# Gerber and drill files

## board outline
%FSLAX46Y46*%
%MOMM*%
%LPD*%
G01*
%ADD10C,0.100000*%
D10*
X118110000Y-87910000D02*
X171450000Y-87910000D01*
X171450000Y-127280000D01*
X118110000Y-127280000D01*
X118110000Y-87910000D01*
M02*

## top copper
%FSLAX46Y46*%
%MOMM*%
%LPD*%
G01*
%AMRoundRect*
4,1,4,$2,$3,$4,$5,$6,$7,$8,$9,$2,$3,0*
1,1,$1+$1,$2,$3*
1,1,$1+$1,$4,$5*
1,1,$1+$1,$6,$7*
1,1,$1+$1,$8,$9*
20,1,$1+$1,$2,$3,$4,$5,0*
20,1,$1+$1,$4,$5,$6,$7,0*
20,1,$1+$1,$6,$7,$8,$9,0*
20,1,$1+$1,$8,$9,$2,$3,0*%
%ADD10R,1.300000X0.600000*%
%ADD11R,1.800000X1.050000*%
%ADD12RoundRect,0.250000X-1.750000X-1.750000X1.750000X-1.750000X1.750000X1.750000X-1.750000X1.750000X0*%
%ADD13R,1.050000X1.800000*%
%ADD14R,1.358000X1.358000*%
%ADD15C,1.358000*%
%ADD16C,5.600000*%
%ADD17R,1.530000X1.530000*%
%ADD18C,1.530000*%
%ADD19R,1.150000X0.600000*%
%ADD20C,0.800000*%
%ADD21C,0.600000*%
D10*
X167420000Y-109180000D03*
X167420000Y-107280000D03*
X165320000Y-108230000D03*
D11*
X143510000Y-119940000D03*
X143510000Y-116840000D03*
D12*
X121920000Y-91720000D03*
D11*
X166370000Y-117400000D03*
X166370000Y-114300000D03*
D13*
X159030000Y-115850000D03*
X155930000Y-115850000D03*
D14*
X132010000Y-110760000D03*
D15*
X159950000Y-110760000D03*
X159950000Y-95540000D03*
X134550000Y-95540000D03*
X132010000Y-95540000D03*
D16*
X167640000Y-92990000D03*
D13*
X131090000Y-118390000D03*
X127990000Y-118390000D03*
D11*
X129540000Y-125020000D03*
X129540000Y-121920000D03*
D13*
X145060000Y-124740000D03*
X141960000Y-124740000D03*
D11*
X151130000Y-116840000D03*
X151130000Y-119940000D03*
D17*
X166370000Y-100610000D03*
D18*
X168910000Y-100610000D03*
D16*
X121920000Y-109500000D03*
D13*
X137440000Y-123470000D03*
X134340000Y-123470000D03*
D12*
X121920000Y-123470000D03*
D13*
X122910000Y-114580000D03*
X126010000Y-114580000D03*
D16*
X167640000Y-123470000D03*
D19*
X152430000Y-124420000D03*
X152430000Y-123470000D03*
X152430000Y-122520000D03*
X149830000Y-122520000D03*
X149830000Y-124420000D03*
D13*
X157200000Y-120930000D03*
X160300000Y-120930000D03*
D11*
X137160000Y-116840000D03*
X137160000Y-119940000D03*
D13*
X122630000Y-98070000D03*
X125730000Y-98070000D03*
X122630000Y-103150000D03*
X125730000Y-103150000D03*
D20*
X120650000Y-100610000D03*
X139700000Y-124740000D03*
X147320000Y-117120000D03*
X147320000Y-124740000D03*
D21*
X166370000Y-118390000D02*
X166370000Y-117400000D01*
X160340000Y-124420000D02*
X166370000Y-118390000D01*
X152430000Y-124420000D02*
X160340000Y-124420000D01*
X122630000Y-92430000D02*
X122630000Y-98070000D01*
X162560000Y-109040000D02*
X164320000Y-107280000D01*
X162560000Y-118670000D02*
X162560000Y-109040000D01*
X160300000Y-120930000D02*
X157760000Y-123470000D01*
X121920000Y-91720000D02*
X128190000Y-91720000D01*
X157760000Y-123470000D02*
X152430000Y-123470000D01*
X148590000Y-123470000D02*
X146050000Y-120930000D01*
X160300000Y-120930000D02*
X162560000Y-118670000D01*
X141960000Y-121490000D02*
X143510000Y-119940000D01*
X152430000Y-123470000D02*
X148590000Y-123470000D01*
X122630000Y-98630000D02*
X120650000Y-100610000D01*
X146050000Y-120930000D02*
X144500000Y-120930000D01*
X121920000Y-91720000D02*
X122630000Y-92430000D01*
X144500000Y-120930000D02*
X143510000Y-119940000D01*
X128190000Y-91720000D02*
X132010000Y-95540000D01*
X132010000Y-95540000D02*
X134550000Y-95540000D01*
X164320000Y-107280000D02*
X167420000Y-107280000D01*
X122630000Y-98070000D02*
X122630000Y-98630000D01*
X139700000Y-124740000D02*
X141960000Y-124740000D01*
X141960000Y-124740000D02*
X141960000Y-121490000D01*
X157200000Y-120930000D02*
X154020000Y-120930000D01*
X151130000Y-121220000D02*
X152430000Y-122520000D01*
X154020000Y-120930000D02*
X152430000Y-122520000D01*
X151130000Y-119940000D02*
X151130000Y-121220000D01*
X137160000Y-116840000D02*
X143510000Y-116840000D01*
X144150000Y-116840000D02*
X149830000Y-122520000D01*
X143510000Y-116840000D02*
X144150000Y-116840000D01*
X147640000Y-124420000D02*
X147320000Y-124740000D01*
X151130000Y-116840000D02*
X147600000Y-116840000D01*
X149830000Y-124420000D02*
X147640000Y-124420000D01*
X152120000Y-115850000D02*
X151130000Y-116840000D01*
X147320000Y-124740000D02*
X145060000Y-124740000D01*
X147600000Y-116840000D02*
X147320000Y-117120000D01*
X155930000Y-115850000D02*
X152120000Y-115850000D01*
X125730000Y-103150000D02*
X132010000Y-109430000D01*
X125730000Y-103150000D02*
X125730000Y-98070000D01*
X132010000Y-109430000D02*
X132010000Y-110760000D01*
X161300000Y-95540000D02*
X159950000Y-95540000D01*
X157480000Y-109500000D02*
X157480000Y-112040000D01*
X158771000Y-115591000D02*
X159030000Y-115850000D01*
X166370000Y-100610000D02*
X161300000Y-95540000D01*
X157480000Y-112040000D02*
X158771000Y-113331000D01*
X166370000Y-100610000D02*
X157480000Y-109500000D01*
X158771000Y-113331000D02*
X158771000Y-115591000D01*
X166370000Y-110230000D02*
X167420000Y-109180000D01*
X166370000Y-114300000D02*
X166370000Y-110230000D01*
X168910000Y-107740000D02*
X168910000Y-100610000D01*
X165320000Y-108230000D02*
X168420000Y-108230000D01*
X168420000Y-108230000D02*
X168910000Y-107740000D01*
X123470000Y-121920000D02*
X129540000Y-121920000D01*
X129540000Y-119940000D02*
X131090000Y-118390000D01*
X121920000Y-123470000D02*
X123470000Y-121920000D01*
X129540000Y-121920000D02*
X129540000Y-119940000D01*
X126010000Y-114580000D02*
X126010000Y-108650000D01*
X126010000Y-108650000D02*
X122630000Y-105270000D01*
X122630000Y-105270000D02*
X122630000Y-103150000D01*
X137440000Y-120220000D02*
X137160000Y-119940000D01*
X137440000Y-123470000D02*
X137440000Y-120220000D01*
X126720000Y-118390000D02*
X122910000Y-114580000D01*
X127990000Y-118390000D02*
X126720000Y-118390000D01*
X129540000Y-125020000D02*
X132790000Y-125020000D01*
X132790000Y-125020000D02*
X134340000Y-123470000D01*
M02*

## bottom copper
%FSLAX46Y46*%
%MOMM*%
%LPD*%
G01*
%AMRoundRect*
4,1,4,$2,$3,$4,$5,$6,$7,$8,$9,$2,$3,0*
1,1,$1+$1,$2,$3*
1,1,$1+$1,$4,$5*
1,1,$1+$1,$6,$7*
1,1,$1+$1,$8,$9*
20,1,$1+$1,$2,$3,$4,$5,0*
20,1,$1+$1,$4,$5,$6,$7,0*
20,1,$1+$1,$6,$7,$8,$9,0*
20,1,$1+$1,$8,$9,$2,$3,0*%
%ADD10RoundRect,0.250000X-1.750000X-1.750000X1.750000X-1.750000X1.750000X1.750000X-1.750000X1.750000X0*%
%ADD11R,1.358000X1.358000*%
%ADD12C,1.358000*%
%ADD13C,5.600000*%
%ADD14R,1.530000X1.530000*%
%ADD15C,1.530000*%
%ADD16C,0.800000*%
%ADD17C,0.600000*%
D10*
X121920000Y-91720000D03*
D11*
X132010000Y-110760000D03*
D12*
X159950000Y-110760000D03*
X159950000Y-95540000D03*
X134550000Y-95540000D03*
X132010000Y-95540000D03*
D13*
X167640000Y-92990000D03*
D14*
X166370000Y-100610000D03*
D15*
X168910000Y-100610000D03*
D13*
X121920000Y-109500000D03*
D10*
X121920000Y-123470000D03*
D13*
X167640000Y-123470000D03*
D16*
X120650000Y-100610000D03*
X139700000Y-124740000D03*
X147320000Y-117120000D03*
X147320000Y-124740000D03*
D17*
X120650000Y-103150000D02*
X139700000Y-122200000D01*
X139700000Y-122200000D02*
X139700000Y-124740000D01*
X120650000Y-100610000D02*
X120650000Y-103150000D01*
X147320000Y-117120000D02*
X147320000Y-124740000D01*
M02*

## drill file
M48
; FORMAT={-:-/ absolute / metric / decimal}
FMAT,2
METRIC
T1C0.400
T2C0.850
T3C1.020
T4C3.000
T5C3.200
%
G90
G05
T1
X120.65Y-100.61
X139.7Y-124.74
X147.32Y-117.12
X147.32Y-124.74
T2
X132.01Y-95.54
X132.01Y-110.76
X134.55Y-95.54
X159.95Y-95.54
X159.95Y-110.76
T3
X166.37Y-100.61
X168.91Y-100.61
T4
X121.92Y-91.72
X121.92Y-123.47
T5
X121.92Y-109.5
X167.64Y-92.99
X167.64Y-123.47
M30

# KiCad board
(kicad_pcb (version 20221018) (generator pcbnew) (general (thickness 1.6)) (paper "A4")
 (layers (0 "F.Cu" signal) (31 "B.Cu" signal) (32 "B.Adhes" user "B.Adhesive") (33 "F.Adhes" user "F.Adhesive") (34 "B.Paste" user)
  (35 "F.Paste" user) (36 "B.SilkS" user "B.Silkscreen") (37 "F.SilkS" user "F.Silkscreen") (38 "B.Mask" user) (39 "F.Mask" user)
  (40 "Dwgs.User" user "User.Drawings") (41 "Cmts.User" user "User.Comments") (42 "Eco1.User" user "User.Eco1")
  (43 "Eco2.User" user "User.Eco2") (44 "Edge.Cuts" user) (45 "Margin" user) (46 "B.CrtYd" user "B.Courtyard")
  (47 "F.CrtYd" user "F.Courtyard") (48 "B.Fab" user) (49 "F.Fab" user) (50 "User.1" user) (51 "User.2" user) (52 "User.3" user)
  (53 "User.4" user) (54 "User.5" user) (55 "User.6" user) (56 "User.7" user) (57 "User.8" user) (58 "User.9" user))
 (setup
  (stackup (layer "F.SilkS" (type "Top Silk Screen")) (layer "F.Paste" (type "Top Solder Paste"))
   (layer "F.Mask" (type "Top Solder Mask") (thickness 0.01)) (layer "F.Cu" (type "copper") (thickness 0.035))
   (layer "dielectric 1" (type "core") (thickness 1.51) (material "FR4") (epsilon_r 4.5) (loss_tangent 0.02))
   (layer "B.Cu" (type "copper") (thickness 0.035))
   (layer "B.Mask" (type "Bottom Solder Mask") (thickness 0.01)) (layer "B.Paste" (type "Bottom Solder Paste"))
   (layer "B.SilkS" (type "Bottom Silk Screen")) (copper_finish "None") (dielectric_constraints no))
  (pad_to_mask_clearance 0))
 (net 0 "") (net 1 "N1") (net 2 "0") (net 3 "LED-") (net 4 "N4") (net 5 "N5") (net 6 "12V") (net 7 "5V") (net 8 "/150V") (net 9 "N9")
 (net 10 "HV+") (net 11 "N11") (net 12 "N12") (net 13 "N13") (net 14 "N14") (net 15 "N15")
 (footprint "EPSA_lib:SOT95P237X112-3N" (layer "F.Cu") (at 166.37 108.23 180)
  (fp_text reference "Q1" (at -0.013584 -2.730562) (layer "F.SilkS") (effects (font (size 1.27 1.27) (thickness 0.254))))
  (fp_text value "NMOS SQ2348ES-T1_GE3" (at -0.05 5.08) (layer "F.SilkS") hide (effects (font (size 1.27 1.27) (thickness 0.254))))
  (pad "1" smd rect (at -1.05 -0.95 270) (size 0.6 1.3) (layers "F.Cu" "F.Paste" "F.Mask") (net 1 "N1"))
  (pad "2" smd rect (at -1.05 0.95 270) (size 0.6 1.3) (layers "F.Cu" "F.Paste" "F.Mask") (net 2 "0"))
  (pad "3" smd rect (at 1.05 0 270) (size 0.6 1.3) (layers "F.Cu" "F.Paste" "F.Mask") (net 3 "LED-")))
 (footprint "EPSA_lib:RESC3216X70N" (layer "F.Cu") (at 143.51 118.39 90)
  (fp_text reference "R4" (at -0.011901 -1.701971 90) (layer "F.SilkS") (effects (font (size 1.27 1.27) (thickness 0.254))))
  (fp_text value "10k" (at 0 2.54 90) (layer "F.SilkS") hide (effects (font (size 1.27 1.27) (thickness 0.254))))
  (pad "1" smd rect (at -1.55 0 90) (size 1.05 1.8) (layers "F.Cu" "F.Paste" "F.Mask") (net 2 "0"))
  (pad "2" smd rect (at 1.55 0 90) (size 1.05 1.8) (layers "F.Cu" "F.Paste" "F.Mask") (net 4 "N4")))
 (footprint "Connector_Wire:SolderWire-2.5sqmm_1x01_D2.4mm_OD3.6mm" (layer "F.Cu") (at 121.92 91.72)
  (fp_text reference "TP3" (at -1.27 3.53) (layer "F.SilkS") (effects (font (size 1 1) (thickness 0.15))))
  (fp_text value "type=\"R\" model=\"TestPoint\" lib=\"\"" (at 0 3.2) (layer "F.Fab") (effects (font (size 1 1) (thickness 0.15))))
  (pad "1" thru_hole roundrect (at 0 0) (size 4 4) (drill 3) (layers "*.Cu" "*.Mask") (roundrect_rratio 0.0625) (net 2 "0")))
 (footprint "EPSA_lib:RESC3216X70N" (layer "F.Cu") (at 166.37 115.85 90)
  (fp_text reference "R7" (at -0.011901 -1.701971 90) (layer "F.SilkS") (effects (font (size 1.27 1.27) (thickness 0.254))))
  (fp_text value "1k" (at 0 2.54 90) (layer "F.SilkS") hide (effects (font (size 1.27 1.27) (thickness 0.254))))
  (pad "1" smd rect (at -1.55 0 90) (size 1.05 1.8) (layers "F.Cu" "F.Paste" "F.Mask") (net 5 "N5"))
  (pad "2" smd rect (at 1.55 0 90) (size 1.05 1.8) (layers "F.Cu" "F.Paste" "F.Mask") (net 1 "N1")))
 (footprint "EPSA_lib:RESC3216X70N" (layer "F.Cu") (at 157.48 115.85 180)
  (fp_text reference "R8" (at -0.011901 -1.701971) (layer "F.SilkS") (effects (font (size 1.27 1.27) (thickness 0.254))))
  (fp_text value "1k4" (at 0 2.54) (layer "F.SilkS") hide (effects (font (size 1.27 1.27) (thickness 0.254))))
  (pad "1" smd rect (at -1.55 0 180) (size 1.05 1.8) (layers "F.Cu" "F.Paste" "F.Mask") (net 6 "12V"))
  (pad "2" smd rect (at 1.55 0 180) (size 1.05 1.8) (layers "F.Cu" "F.Paste" "F.Mask") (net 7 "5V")))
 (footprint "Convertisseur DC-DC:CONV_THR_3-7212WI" (layer "F.Cu") (at 146.05 103.15 180)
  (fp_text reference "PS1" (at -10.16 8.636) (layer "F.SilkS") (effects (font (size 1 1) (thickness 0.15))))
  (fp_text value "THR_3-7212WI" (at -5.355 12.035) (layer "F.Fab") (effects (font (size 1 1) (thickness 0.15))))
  (pad "1" thru_hole rect (at 14.04 -7.61 180) (size 1.358 1.358) (drill 0.85) (layers "*.Cu" "*.Mask") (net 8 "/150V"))
  (pad "12" thru_hole circle (at -13.9 -7.61 180) (size 1.358 1.358) (drill 0.85) (layers "*.Cu" "*.Mask") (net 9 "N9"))
  (pad "13" thru_hole circle (at -13.9 7.61 180) (size 1.358 1.358) (drill 0.85) (layers "*.Cu" "*.Mask") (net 6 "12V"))
  (pad "23" thru_hole circle (at 11.5 7.61 180) (size 1.358 1.358) (drill 0.85) (layers "*.Cu" "*.Mask") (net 2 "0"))
  (pad "24" thru_hole circle (at 14.04 7.61 180) (size 1.358 1.358) (drill 0.85) (layers "*.Cu" "*.Mask") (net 2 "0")))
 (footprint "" (layer "F.Cu") (at 167.64 92.99)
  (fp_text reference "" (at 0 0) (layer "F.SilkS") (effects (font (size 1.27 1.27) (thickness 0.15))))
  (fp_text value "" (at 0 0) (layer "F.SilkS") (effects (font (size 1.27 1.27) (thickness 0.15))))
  (pad "1" thru_hole circle (at 0 0) (size 5.6 5.6) (drill 3.2) (layers "*.Cu" "*.Mask")))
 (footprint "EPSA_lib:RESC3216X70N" (layer "F.Cu") (at 129.54 118.39 180)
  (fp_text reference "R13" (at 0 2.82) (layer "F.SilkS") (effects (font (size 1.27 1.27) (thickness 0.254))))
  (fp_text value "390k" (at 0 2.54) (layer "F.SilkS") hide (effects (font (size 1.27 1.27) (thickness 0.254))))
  (pad "1" smd rect (at -1.55 0 180) (size 1.05 1.8) (layers "F.Cu" "F.Paste" "F.Mask") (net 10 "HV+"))
  (pad "2" smd rect (at 1.55 0 180) (size 1.05 1.8) (layers "F.Cu" "F.Paste" "F.Mask") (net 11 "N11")))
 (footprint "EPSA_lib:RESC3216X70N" (layer "F.Cu") (at 129.54 123.47 90)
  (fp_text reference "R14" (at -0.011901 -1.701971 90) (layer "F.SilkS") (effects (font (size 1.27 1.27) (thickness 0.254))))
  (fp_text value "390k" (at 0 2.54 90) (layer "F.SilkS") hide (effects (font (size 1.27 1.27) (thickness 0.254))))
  (pad "1" smd rect (at -1.55 0 90) (size 1.05 1.8) (layers "F.Cu" "F.Paste" "F.Mask") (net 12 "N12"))
  (pad "2" smd rect (at 1.55 0 90) (size 1.05 1.8) (layers "F.Cu" "F.Paste" "F.Mask") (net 10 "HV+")))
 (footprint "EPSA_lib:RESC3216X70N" (layer "F.Cu") (at 143.51 124.74 180)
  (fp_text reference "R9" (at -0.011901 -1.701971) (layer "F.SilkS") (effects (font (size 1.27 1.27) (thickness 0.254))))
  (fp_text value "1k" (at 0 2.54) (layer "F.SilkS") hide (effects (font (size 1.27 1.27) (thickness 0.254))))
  (pad "1" smd rect (at -1.55 0 180) (size 1.05 1.8) (layers "F.Cu" "F.Paste" "F.Mask") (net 7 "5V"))
  (pad "2" smd rect (at 1.55 0 180) (size 1.05 1.8) (layers "F.Cu" "F.Paste" "F.Mask") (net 2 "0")))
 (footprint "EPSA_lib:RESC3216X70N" (layer "F.Cu") (at 151.13 118.39 -90)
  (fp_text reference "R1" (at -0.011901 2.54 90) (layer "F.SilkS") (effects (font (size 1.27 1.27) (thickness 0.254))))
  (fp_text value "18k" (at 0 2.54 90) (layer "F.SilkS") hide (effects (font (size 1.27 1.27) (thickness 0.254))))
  (pad "1" smd rect (at -1.55 0 270) (size 1.05 1.8) (layers "F.Cu" "F.Paste" "F.Mask") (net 7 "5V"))
  (pad "2" smd rect (at 1.55 0 270) (size 1.05 1.8) (layers "F.Cu" "F.Paste" "F.Mask") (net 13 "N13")))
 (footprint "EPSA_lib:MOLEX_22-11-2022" (layer "F.Cu") (at 166.37 100.61)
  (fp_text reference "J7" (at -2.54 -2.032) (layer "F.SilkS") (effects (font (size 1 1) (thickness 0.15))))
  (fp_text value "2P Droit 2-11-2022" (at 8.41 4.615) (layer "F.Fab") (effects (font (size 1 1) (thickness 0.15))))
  (pad "1" thru_hole rect (at 0 0) (size 1.53 1.53) (drill 1.02) (layers "*.Cu" "*.Mask") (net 6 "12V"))
  (pad "2" thru_hole circle (at 2.54 0) (size 1.53 1.53) (drill 1.02) (layers "*.Cu" "*.Mask") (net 3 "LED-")))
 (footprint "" (layer "F.Cu") (at 121.92 109.5)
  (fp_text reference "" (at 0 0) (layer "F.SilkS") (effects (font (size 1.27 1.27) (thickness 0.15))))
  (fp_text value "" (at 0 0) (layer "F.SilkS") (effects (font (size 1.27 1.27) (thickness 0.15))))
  (pad "1" thru_hole circle (at 0 0) (size 5.6 5.6) (drill 3.2) (layers "*.Cu" "*.Mask")))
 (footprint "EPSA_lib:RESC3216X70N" (layer "F.Cu") (at 135.89 123.47 180)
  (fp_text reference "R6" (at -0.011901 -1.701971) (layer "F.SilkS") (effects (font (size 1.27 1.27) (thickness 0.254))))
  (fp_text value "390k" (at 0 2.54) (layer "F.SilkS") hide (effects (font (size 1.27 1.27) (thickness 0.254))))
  (pad "1" smd rect (at -1.55 0 180) (size 1.05 1.8) (layers "F.Cu" "F.Paste" "F.Mask") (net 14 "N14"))
  (pad "2" smd rect (at 1.55 0 180) (size 1.05 1.8) (layers "F.Cu" "F.Paste" "F.Mask") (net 12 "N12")))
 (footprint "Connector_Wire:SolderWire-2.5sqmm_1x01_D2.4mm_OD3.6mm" (layer "F.Cu") (at 121.92 123.47)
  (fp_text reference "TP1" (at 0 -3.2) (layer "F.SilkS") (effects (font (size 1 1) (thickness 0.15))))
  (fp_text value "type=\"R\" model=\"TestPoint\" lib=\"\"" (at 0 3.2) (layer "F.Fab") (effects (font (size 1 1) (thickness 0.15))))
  (pad "1" thru_hole roundrect (at 0 0) (size 4 4) (drill 3) (layers "*.Cu" "*.Mask") (roundrect_rratio 0.0625) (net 10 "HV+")))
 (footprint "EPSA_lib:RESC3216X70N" (layer "F.Cu") (at 124.46 114.58)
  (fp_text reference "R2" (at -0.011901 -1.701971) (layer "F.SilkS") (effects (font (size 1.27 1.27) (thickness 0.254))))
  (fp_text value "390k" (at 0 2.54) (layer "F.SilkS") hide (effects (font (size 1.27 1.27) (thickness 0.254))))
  (pad "1" smd rect (at -1.55 0) (size 1.05 1.8) (layers "F.Cu" "F.Paste" "F.Mask") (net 11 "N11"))
  (pad "2" smd rect (at 1.55 0) (size 1.05 1.8) (layers "F.Cu" "F.Paste" "F.Mask") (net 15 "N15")))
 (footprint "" (layer "F.Cu") (at 167.64 123.47)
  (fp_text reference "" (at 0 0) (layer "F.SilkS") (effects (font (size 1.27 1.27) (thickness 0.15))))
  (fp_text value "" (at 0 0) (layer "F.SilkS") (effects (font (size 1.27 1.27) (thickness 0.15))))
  (pad "1" thru_hole circle (at 0 0) (size 5.6 5.6) (drill 3.2) (layers "*.Cu" "*.Mask")))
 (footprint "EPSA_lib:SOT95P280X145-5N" (layer "F.Cu") (at 151.13 123.47 180)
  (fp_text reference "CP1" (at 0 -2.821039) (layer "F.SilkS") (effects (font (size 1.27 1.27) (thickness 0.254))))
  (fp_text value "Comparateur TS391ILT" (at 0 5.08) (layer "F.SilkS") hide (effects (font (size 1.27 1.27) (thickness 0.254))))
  (pad "1" smd rect (at -1.3 -0.95 270) (size 0.6 1.15) (layers "F.Cu" "F.Paste" "F.Mask") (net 5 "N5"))
  (pad "2" smd rect (at -1.3 0 270) (size 0.6 1.15) (layers "F.Cu" "F.Paste" "F.Mask") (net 2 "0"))
  (pad "3" smd rect (at -1.3 0.95 270) (size 0.6 1.15) (layers "F.Cu" "F.Paste" "F.Mask") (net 13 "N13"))
  (pad "4" smd rect (at 1.3 0.95 270) (size 0.6 1.15) (layers "F.Cu" "F.Paste" "F.Mask") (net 4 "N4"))
  (pad "5" smd rect (at 1.3 -0.95 270) (size 0.6 1.15) (layers "F.Cu" "F.Paste" "F.Mask") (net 7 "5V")))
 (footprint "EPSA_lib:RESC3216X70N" (layer "F.Cu") (at 158.75 120.93)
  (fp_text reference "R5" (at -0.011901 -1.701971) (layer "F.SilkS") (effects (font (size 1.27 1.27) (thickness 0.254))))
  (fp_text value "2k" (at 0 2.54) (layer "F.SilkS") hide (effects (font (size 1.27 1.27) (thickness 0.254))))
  (pad "1" smd rect (at -1.55 0) (size 1.05 1.8) (layers "F.Cu" "F.Paste" "F.Mask") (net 13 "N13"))
  (pad "2" smd rect (at 1.55 0) (size 1.05 1.8) (layers "F.Cu" "F.Paste" "F.Mask") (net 2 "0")))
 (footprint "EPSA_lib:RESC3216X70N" (layer "F.Cu") (at 137.16 118.39 -90)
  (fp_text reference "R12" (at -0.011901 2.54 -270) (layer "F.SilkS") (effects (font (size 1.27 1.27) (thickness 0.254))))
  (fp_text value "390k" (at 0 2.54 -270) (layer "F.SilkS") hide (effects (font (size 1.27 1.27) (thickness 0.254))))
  (pad "1" smd rect (at -1.55 0 270) (size 1.05 1.8) (layers "F.Cu" "F.Paste" "F.Mask") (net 4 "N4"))
  (pad "2" smd rect (at 1.55 0 270) (size 1.05 1.8) (layers "F.Cu" "F.Paste" "F.Mask") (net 14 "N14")))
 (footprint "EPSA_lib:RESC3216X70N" (layer "F.Cu") (at 124.18 98.07)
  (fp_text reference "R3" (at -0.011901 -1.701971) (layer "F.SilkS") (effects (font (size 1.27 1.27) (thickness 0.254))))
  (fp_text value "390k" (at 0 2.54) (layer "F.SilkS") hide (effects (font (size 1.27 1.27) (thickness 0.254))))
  (pad "1" smd rect (at -1.55 0) (size 1.05 1.8) (layers "F.Cu" "F.Paste" "F.Mask") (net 2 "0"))
  (pad "2" smd rect (at 1.55 0) (size 1.05 1.8) (layers "F.Cu" "F.Paste" "F.Mask") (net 8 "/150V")))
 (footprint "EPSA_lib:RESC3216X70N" (layer "F.Cu") (at 124.18 103.15)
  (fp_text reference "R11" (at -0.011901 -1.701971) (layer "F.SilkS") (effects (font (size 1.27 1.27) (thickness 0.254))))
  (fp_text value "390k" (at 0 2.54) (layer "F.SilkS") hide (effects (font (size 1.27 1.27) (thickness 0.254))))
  (pad "1" smd rect (at -1.55 0) (size 1.05 1.8) (layers "F.Cu" "F.Paste" "F.Mask") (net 15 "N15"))
  (pad "2" smd rect (at 1.55 0) (size 1.05 1.8) (layers "F.Cu" "F.Paste" "F.Mask") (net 8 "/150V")))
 (gr_rect (start 118.11 87.91) (end 171.45 127.28) (stroke (width 0.1) (type default)) (fill none) (layer "Edge.Cuts"))
 (segment (start 166.37 118.39) (end 166.37 117.4) (width 0.6) (layer "F.Cu") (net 5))
 (segment (start 160.34 124.42) (end 166.37 118.39) (width 0.6) (layer "F.Cu") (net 5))
 (segment (start 152.43 124.42) (end 160.34 124.42) (width 0.6) (layer "F.Cu") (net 5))
 (segment (start 122.63 92.43) (end 122.63 98.07) (width 0.6) (layer "F.Cu") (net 2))
 (segment (start 162.56 109.04) (end 164.32 107.28) (width 0.6) (layer "F.Cu") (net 2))
 (segment (start 162.56 118.67) (end 162.56 109.04) (width 0.6) (layer "F.Cu") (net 2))
 (segment (start 160.3 120.93) (end 157.76 123.47) (width 0.6) (layer "F.Cu") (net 2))
 (segment (start 121.92 91.72) (end 128.19 91.72) (width 0.6) (layer "F.Cu") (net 2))
 (segment (start 157.76 123.47) (end 152.43 123.47) (width 0.6) (layer "F.Cu") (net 2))
 (segment (start 148.59 123.47) (end 146.05 120.93) (width 0.6) (layer "F.Cu") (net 2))
 (segment (start 160.3 120.93) (end 162.56 118.67) (width 0.6) (layer "F.Cu") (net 2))
 (segment (start 141.96 121.49) (end 143.51 119.94) (width 0.6) (layer "F.Cu") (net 2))
 (segment (start 152.43 123.47) (end 148.59 123.47) (width 0.6) (layer "F.Cu") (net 2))
 (segment (start 122.63 98.63) (end 120.65 100.61) (width 0.6) (layer "F.Cu") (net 2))
 (segment (start 146.05 120.93) (end 144.5 120.93) (width 0.6) (layer "F.Cu") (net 2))
 (segment (start 121.92 91.72) (end 122.63 92.43) (width 0.6) (layer "F.Cu") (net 2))
 (segment (start 144.5 120.93) (end 143.51 119.94) (width 0.6) (layer "F.Cu") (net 2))
 (segment (start 128.19 91.72) (end 132.01 95.54) (width 0.6) (layer "F.Cu") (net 2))
 (segment (start 132.01 95.54) (end 134.55 95.54) (width 0.6) (layer "F.Cu") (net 2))
 (segment (start 164.32 107.28) (end 167.42 107.28) (width 0.6) (layer "F.Cu") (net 2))
 (segment (start 122.63 98.07) (end 122.63 98.63) (width 0.6) (layer "F.Cu") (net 2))
 (segment (start 139.7 124.74) (end 141.96 124.74) (width 0.6) (layer "F.Cu") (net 2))
 (segment (start 141.96 124.74) (end 141.96 121.49) (width 0.6) (layer "F.Cu") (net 2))
 (via (at 120.65 100.61) (size 0.8) (drill 0.4) (layers "F.Cu" "B.Cu") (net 2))
 (via (at 139.7 124.74) (size 0.8) (drill 0.4) (layers "F.Cu" "B.Cu") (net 2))
 (segment (start 120.65 103.15) (end 139.7 122.2) (width 0.6) (layer "B.Cu") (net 2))
 (segment (start 139.7 122.2) (end 139.7 124.74) (width 0.6) (layer "B.Cu") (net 2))
 (segment (start 120.65 100.61) (end 120.65 103.15) (width 0.6) (layer "B.Cu") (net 2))
 (segment (start 157.2 120.93) (end 154.02 120.93) (width 0.6) (layer "F.Cu") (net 13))
 (segment (start 151.13 121.22) (end 152.43 122.52) (width 0.6) (layer "F.Cu") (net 13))
 (segment (start 154.02 120.93) (end 152.43 122.52) (width 0.6) (layer "F.Cu") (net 13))
 (segment (start 151.13 119.94) (end 151.13 121.22) (width 0.6) (layer "F.Cu") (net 13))
 (segment (start 137.16 116.84) (end 143.51 116.84) (width 0.6) (layer "F.Cu") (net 4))
 (segment (start 144.15 116.84) (end 149.83 122.52) (width 0.6) (layer "F.Cu") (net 4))
 (segment (start 143.51 116.84) (end 144.15 116.84) (width 0.6) (layer "F.Cu") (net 4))
 (segment (start 147.64 124.42) (end 147.32 124.74) (width 0.6) (layer "F.Cu") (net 7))
 (segment (start 151.13 116.84) (end 147.6 116.84) (width 0.6) (layer "F.Cu") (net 7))
 (segment (start 149.83 124.42) (end 147.64 124.42) (width 0.6) (layer "F.Cu") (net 7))
 (segment (start 152.12 115.85) (end 151.13 116.84) (width 0.6) (layer "F.Cu") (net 7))
 (segment (start 147.32 124.74) (end 145.06 124.74) (width 0.6) (layer "F.Cu") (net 7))
 (segment (start 147.6 116.84) (end 147.32 117.12) (width 0.6) (layer "F.Cu") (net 7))
 (segment (start 155.93 115.85) (end 152.12 115.85) (width 0.6) (layer "F.Cu") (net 7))
 (via (at 147.32 117.12) (size 0.8) (drill 0.4) (layers "F.Cu" "B.Cu") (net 7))
 (via (at 147.32 124.74) (size 0.8) (drill 0.4) (layers "F.Cu" "B.Cu") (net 7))
 (segment (start 147.32 117.12) (end 147.32 124.74) (width 0.6) (layer "B.Cu") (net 7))
 (segment (start 125.73 103.15) (end 132.01 109.43) (width 0.6) (layer "F.Cu") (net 8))
 (segment (start 125.73 103.15) (end 125.73 98.07) (width 0.6) (layer "F.Cu") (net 8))
 (segment (start 132.01 109.43) (end 132.01 110.76) (width 0.6) (layer "F.Cu") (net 8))
 (segment (start 161.3 95.54) (end 159.95 95.54) (width 0.6) (layer "F.Cu") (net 6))
 (segment (start 157.48 109.5) (end 157.48 112.04) (width 0.6) (layer "F.Cu") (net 6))
 (segment (start 158.771 115.591) (end 159.03 115.85) (width 0.6) (layer "F.Cu") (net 6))
 (segment (start 166.37 100.61) (end 161.3 95.54) (width 0.6) (layer "F.Cu") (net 6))
 (segment (start 157.48 112.04) (end 158.771 113.331) (width 0.6) (layer "F.Cu") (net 6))
 (segment (start 166.37 100.61) (end 157.48 109.5) (width 0.6) (layer "F.Cu") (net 6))
 (segment (start 158.771 113.331) (end 158.771 115.591) (width 0.6) (layer "F.Cu") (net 6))
 (segment (start 166.37 110.23) (end 167.42 109.18) (width 0.6) (layer "F.Cu") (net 1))
 (segment (start 166.37 114.3) (end 166.37 110.23) (width 0.6) (layer "F.Cu") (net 1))
 (segment (start 168.91 107.74) (end 168.91 100.61) (width 0.6) (layer "F.Cu") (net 3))
 (segment (start 165.32 108.23) (end 168.42 108.23) (width 0.6) (layer "F.Cu") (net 3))
 (segment (start 168.42 108.23) (end 168.91 107.74) (width 0.6) (layer "F.Cu") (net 3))
 (segment (start 123.47 121.92) (end 129.54 121.92) (width 0.6) (layer "F.Cu") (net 10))
 (segment (start 129.54 119.94) (end 131.09 118.39) (width 0.6) (layer "F.Cu") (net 10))
 (segment (start 121.92 123.47) (end 123.47 121.92) (width 0.6) (layer "F.Cu") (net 10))
 (segment (start 129.54 121.92) (end 129.54 119.94) (width 0.6) (layer "F.Cu") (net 10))
 (segment (start 126.01 114.58) (end 126.01 108.65) (width 0.6) (layer "F.Cu") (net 15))
 (segment (start 126.01 108.65) (end 122.63 105.27) (width 0.6) (layer "F.Cu") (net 15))
 (segment (start 122.63 105.27) (end 122.63 103.15) (width 0.6) (layer "F.Cu") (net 15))
 (segment (start 137.44 120.22) (end 137.16 119.94) (width 0.6) (layer "F.Cu") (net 14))
 (segment (start 137.44 123.47) (end 137.44 120.22) (width 0.6) (layer "F.Cu") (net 14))
 (segment (start 126.72 118.39) (end 122.91 114.58) (width 0.6) (layer "F.Cu") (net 11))
 (segment (start 127.99 118.39) (end 126.72 118.39) (width 0.6) (layer "F.Cu") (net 11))
 (segment (start 129.54 125.02) (end 132.79 125.02) (width 0.6) (layer "F.Cu") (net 12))
 (segment (start 132.79 125.02) (end 134.34 123.47) (width 0.6) (layer "F.Cu") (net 12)))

